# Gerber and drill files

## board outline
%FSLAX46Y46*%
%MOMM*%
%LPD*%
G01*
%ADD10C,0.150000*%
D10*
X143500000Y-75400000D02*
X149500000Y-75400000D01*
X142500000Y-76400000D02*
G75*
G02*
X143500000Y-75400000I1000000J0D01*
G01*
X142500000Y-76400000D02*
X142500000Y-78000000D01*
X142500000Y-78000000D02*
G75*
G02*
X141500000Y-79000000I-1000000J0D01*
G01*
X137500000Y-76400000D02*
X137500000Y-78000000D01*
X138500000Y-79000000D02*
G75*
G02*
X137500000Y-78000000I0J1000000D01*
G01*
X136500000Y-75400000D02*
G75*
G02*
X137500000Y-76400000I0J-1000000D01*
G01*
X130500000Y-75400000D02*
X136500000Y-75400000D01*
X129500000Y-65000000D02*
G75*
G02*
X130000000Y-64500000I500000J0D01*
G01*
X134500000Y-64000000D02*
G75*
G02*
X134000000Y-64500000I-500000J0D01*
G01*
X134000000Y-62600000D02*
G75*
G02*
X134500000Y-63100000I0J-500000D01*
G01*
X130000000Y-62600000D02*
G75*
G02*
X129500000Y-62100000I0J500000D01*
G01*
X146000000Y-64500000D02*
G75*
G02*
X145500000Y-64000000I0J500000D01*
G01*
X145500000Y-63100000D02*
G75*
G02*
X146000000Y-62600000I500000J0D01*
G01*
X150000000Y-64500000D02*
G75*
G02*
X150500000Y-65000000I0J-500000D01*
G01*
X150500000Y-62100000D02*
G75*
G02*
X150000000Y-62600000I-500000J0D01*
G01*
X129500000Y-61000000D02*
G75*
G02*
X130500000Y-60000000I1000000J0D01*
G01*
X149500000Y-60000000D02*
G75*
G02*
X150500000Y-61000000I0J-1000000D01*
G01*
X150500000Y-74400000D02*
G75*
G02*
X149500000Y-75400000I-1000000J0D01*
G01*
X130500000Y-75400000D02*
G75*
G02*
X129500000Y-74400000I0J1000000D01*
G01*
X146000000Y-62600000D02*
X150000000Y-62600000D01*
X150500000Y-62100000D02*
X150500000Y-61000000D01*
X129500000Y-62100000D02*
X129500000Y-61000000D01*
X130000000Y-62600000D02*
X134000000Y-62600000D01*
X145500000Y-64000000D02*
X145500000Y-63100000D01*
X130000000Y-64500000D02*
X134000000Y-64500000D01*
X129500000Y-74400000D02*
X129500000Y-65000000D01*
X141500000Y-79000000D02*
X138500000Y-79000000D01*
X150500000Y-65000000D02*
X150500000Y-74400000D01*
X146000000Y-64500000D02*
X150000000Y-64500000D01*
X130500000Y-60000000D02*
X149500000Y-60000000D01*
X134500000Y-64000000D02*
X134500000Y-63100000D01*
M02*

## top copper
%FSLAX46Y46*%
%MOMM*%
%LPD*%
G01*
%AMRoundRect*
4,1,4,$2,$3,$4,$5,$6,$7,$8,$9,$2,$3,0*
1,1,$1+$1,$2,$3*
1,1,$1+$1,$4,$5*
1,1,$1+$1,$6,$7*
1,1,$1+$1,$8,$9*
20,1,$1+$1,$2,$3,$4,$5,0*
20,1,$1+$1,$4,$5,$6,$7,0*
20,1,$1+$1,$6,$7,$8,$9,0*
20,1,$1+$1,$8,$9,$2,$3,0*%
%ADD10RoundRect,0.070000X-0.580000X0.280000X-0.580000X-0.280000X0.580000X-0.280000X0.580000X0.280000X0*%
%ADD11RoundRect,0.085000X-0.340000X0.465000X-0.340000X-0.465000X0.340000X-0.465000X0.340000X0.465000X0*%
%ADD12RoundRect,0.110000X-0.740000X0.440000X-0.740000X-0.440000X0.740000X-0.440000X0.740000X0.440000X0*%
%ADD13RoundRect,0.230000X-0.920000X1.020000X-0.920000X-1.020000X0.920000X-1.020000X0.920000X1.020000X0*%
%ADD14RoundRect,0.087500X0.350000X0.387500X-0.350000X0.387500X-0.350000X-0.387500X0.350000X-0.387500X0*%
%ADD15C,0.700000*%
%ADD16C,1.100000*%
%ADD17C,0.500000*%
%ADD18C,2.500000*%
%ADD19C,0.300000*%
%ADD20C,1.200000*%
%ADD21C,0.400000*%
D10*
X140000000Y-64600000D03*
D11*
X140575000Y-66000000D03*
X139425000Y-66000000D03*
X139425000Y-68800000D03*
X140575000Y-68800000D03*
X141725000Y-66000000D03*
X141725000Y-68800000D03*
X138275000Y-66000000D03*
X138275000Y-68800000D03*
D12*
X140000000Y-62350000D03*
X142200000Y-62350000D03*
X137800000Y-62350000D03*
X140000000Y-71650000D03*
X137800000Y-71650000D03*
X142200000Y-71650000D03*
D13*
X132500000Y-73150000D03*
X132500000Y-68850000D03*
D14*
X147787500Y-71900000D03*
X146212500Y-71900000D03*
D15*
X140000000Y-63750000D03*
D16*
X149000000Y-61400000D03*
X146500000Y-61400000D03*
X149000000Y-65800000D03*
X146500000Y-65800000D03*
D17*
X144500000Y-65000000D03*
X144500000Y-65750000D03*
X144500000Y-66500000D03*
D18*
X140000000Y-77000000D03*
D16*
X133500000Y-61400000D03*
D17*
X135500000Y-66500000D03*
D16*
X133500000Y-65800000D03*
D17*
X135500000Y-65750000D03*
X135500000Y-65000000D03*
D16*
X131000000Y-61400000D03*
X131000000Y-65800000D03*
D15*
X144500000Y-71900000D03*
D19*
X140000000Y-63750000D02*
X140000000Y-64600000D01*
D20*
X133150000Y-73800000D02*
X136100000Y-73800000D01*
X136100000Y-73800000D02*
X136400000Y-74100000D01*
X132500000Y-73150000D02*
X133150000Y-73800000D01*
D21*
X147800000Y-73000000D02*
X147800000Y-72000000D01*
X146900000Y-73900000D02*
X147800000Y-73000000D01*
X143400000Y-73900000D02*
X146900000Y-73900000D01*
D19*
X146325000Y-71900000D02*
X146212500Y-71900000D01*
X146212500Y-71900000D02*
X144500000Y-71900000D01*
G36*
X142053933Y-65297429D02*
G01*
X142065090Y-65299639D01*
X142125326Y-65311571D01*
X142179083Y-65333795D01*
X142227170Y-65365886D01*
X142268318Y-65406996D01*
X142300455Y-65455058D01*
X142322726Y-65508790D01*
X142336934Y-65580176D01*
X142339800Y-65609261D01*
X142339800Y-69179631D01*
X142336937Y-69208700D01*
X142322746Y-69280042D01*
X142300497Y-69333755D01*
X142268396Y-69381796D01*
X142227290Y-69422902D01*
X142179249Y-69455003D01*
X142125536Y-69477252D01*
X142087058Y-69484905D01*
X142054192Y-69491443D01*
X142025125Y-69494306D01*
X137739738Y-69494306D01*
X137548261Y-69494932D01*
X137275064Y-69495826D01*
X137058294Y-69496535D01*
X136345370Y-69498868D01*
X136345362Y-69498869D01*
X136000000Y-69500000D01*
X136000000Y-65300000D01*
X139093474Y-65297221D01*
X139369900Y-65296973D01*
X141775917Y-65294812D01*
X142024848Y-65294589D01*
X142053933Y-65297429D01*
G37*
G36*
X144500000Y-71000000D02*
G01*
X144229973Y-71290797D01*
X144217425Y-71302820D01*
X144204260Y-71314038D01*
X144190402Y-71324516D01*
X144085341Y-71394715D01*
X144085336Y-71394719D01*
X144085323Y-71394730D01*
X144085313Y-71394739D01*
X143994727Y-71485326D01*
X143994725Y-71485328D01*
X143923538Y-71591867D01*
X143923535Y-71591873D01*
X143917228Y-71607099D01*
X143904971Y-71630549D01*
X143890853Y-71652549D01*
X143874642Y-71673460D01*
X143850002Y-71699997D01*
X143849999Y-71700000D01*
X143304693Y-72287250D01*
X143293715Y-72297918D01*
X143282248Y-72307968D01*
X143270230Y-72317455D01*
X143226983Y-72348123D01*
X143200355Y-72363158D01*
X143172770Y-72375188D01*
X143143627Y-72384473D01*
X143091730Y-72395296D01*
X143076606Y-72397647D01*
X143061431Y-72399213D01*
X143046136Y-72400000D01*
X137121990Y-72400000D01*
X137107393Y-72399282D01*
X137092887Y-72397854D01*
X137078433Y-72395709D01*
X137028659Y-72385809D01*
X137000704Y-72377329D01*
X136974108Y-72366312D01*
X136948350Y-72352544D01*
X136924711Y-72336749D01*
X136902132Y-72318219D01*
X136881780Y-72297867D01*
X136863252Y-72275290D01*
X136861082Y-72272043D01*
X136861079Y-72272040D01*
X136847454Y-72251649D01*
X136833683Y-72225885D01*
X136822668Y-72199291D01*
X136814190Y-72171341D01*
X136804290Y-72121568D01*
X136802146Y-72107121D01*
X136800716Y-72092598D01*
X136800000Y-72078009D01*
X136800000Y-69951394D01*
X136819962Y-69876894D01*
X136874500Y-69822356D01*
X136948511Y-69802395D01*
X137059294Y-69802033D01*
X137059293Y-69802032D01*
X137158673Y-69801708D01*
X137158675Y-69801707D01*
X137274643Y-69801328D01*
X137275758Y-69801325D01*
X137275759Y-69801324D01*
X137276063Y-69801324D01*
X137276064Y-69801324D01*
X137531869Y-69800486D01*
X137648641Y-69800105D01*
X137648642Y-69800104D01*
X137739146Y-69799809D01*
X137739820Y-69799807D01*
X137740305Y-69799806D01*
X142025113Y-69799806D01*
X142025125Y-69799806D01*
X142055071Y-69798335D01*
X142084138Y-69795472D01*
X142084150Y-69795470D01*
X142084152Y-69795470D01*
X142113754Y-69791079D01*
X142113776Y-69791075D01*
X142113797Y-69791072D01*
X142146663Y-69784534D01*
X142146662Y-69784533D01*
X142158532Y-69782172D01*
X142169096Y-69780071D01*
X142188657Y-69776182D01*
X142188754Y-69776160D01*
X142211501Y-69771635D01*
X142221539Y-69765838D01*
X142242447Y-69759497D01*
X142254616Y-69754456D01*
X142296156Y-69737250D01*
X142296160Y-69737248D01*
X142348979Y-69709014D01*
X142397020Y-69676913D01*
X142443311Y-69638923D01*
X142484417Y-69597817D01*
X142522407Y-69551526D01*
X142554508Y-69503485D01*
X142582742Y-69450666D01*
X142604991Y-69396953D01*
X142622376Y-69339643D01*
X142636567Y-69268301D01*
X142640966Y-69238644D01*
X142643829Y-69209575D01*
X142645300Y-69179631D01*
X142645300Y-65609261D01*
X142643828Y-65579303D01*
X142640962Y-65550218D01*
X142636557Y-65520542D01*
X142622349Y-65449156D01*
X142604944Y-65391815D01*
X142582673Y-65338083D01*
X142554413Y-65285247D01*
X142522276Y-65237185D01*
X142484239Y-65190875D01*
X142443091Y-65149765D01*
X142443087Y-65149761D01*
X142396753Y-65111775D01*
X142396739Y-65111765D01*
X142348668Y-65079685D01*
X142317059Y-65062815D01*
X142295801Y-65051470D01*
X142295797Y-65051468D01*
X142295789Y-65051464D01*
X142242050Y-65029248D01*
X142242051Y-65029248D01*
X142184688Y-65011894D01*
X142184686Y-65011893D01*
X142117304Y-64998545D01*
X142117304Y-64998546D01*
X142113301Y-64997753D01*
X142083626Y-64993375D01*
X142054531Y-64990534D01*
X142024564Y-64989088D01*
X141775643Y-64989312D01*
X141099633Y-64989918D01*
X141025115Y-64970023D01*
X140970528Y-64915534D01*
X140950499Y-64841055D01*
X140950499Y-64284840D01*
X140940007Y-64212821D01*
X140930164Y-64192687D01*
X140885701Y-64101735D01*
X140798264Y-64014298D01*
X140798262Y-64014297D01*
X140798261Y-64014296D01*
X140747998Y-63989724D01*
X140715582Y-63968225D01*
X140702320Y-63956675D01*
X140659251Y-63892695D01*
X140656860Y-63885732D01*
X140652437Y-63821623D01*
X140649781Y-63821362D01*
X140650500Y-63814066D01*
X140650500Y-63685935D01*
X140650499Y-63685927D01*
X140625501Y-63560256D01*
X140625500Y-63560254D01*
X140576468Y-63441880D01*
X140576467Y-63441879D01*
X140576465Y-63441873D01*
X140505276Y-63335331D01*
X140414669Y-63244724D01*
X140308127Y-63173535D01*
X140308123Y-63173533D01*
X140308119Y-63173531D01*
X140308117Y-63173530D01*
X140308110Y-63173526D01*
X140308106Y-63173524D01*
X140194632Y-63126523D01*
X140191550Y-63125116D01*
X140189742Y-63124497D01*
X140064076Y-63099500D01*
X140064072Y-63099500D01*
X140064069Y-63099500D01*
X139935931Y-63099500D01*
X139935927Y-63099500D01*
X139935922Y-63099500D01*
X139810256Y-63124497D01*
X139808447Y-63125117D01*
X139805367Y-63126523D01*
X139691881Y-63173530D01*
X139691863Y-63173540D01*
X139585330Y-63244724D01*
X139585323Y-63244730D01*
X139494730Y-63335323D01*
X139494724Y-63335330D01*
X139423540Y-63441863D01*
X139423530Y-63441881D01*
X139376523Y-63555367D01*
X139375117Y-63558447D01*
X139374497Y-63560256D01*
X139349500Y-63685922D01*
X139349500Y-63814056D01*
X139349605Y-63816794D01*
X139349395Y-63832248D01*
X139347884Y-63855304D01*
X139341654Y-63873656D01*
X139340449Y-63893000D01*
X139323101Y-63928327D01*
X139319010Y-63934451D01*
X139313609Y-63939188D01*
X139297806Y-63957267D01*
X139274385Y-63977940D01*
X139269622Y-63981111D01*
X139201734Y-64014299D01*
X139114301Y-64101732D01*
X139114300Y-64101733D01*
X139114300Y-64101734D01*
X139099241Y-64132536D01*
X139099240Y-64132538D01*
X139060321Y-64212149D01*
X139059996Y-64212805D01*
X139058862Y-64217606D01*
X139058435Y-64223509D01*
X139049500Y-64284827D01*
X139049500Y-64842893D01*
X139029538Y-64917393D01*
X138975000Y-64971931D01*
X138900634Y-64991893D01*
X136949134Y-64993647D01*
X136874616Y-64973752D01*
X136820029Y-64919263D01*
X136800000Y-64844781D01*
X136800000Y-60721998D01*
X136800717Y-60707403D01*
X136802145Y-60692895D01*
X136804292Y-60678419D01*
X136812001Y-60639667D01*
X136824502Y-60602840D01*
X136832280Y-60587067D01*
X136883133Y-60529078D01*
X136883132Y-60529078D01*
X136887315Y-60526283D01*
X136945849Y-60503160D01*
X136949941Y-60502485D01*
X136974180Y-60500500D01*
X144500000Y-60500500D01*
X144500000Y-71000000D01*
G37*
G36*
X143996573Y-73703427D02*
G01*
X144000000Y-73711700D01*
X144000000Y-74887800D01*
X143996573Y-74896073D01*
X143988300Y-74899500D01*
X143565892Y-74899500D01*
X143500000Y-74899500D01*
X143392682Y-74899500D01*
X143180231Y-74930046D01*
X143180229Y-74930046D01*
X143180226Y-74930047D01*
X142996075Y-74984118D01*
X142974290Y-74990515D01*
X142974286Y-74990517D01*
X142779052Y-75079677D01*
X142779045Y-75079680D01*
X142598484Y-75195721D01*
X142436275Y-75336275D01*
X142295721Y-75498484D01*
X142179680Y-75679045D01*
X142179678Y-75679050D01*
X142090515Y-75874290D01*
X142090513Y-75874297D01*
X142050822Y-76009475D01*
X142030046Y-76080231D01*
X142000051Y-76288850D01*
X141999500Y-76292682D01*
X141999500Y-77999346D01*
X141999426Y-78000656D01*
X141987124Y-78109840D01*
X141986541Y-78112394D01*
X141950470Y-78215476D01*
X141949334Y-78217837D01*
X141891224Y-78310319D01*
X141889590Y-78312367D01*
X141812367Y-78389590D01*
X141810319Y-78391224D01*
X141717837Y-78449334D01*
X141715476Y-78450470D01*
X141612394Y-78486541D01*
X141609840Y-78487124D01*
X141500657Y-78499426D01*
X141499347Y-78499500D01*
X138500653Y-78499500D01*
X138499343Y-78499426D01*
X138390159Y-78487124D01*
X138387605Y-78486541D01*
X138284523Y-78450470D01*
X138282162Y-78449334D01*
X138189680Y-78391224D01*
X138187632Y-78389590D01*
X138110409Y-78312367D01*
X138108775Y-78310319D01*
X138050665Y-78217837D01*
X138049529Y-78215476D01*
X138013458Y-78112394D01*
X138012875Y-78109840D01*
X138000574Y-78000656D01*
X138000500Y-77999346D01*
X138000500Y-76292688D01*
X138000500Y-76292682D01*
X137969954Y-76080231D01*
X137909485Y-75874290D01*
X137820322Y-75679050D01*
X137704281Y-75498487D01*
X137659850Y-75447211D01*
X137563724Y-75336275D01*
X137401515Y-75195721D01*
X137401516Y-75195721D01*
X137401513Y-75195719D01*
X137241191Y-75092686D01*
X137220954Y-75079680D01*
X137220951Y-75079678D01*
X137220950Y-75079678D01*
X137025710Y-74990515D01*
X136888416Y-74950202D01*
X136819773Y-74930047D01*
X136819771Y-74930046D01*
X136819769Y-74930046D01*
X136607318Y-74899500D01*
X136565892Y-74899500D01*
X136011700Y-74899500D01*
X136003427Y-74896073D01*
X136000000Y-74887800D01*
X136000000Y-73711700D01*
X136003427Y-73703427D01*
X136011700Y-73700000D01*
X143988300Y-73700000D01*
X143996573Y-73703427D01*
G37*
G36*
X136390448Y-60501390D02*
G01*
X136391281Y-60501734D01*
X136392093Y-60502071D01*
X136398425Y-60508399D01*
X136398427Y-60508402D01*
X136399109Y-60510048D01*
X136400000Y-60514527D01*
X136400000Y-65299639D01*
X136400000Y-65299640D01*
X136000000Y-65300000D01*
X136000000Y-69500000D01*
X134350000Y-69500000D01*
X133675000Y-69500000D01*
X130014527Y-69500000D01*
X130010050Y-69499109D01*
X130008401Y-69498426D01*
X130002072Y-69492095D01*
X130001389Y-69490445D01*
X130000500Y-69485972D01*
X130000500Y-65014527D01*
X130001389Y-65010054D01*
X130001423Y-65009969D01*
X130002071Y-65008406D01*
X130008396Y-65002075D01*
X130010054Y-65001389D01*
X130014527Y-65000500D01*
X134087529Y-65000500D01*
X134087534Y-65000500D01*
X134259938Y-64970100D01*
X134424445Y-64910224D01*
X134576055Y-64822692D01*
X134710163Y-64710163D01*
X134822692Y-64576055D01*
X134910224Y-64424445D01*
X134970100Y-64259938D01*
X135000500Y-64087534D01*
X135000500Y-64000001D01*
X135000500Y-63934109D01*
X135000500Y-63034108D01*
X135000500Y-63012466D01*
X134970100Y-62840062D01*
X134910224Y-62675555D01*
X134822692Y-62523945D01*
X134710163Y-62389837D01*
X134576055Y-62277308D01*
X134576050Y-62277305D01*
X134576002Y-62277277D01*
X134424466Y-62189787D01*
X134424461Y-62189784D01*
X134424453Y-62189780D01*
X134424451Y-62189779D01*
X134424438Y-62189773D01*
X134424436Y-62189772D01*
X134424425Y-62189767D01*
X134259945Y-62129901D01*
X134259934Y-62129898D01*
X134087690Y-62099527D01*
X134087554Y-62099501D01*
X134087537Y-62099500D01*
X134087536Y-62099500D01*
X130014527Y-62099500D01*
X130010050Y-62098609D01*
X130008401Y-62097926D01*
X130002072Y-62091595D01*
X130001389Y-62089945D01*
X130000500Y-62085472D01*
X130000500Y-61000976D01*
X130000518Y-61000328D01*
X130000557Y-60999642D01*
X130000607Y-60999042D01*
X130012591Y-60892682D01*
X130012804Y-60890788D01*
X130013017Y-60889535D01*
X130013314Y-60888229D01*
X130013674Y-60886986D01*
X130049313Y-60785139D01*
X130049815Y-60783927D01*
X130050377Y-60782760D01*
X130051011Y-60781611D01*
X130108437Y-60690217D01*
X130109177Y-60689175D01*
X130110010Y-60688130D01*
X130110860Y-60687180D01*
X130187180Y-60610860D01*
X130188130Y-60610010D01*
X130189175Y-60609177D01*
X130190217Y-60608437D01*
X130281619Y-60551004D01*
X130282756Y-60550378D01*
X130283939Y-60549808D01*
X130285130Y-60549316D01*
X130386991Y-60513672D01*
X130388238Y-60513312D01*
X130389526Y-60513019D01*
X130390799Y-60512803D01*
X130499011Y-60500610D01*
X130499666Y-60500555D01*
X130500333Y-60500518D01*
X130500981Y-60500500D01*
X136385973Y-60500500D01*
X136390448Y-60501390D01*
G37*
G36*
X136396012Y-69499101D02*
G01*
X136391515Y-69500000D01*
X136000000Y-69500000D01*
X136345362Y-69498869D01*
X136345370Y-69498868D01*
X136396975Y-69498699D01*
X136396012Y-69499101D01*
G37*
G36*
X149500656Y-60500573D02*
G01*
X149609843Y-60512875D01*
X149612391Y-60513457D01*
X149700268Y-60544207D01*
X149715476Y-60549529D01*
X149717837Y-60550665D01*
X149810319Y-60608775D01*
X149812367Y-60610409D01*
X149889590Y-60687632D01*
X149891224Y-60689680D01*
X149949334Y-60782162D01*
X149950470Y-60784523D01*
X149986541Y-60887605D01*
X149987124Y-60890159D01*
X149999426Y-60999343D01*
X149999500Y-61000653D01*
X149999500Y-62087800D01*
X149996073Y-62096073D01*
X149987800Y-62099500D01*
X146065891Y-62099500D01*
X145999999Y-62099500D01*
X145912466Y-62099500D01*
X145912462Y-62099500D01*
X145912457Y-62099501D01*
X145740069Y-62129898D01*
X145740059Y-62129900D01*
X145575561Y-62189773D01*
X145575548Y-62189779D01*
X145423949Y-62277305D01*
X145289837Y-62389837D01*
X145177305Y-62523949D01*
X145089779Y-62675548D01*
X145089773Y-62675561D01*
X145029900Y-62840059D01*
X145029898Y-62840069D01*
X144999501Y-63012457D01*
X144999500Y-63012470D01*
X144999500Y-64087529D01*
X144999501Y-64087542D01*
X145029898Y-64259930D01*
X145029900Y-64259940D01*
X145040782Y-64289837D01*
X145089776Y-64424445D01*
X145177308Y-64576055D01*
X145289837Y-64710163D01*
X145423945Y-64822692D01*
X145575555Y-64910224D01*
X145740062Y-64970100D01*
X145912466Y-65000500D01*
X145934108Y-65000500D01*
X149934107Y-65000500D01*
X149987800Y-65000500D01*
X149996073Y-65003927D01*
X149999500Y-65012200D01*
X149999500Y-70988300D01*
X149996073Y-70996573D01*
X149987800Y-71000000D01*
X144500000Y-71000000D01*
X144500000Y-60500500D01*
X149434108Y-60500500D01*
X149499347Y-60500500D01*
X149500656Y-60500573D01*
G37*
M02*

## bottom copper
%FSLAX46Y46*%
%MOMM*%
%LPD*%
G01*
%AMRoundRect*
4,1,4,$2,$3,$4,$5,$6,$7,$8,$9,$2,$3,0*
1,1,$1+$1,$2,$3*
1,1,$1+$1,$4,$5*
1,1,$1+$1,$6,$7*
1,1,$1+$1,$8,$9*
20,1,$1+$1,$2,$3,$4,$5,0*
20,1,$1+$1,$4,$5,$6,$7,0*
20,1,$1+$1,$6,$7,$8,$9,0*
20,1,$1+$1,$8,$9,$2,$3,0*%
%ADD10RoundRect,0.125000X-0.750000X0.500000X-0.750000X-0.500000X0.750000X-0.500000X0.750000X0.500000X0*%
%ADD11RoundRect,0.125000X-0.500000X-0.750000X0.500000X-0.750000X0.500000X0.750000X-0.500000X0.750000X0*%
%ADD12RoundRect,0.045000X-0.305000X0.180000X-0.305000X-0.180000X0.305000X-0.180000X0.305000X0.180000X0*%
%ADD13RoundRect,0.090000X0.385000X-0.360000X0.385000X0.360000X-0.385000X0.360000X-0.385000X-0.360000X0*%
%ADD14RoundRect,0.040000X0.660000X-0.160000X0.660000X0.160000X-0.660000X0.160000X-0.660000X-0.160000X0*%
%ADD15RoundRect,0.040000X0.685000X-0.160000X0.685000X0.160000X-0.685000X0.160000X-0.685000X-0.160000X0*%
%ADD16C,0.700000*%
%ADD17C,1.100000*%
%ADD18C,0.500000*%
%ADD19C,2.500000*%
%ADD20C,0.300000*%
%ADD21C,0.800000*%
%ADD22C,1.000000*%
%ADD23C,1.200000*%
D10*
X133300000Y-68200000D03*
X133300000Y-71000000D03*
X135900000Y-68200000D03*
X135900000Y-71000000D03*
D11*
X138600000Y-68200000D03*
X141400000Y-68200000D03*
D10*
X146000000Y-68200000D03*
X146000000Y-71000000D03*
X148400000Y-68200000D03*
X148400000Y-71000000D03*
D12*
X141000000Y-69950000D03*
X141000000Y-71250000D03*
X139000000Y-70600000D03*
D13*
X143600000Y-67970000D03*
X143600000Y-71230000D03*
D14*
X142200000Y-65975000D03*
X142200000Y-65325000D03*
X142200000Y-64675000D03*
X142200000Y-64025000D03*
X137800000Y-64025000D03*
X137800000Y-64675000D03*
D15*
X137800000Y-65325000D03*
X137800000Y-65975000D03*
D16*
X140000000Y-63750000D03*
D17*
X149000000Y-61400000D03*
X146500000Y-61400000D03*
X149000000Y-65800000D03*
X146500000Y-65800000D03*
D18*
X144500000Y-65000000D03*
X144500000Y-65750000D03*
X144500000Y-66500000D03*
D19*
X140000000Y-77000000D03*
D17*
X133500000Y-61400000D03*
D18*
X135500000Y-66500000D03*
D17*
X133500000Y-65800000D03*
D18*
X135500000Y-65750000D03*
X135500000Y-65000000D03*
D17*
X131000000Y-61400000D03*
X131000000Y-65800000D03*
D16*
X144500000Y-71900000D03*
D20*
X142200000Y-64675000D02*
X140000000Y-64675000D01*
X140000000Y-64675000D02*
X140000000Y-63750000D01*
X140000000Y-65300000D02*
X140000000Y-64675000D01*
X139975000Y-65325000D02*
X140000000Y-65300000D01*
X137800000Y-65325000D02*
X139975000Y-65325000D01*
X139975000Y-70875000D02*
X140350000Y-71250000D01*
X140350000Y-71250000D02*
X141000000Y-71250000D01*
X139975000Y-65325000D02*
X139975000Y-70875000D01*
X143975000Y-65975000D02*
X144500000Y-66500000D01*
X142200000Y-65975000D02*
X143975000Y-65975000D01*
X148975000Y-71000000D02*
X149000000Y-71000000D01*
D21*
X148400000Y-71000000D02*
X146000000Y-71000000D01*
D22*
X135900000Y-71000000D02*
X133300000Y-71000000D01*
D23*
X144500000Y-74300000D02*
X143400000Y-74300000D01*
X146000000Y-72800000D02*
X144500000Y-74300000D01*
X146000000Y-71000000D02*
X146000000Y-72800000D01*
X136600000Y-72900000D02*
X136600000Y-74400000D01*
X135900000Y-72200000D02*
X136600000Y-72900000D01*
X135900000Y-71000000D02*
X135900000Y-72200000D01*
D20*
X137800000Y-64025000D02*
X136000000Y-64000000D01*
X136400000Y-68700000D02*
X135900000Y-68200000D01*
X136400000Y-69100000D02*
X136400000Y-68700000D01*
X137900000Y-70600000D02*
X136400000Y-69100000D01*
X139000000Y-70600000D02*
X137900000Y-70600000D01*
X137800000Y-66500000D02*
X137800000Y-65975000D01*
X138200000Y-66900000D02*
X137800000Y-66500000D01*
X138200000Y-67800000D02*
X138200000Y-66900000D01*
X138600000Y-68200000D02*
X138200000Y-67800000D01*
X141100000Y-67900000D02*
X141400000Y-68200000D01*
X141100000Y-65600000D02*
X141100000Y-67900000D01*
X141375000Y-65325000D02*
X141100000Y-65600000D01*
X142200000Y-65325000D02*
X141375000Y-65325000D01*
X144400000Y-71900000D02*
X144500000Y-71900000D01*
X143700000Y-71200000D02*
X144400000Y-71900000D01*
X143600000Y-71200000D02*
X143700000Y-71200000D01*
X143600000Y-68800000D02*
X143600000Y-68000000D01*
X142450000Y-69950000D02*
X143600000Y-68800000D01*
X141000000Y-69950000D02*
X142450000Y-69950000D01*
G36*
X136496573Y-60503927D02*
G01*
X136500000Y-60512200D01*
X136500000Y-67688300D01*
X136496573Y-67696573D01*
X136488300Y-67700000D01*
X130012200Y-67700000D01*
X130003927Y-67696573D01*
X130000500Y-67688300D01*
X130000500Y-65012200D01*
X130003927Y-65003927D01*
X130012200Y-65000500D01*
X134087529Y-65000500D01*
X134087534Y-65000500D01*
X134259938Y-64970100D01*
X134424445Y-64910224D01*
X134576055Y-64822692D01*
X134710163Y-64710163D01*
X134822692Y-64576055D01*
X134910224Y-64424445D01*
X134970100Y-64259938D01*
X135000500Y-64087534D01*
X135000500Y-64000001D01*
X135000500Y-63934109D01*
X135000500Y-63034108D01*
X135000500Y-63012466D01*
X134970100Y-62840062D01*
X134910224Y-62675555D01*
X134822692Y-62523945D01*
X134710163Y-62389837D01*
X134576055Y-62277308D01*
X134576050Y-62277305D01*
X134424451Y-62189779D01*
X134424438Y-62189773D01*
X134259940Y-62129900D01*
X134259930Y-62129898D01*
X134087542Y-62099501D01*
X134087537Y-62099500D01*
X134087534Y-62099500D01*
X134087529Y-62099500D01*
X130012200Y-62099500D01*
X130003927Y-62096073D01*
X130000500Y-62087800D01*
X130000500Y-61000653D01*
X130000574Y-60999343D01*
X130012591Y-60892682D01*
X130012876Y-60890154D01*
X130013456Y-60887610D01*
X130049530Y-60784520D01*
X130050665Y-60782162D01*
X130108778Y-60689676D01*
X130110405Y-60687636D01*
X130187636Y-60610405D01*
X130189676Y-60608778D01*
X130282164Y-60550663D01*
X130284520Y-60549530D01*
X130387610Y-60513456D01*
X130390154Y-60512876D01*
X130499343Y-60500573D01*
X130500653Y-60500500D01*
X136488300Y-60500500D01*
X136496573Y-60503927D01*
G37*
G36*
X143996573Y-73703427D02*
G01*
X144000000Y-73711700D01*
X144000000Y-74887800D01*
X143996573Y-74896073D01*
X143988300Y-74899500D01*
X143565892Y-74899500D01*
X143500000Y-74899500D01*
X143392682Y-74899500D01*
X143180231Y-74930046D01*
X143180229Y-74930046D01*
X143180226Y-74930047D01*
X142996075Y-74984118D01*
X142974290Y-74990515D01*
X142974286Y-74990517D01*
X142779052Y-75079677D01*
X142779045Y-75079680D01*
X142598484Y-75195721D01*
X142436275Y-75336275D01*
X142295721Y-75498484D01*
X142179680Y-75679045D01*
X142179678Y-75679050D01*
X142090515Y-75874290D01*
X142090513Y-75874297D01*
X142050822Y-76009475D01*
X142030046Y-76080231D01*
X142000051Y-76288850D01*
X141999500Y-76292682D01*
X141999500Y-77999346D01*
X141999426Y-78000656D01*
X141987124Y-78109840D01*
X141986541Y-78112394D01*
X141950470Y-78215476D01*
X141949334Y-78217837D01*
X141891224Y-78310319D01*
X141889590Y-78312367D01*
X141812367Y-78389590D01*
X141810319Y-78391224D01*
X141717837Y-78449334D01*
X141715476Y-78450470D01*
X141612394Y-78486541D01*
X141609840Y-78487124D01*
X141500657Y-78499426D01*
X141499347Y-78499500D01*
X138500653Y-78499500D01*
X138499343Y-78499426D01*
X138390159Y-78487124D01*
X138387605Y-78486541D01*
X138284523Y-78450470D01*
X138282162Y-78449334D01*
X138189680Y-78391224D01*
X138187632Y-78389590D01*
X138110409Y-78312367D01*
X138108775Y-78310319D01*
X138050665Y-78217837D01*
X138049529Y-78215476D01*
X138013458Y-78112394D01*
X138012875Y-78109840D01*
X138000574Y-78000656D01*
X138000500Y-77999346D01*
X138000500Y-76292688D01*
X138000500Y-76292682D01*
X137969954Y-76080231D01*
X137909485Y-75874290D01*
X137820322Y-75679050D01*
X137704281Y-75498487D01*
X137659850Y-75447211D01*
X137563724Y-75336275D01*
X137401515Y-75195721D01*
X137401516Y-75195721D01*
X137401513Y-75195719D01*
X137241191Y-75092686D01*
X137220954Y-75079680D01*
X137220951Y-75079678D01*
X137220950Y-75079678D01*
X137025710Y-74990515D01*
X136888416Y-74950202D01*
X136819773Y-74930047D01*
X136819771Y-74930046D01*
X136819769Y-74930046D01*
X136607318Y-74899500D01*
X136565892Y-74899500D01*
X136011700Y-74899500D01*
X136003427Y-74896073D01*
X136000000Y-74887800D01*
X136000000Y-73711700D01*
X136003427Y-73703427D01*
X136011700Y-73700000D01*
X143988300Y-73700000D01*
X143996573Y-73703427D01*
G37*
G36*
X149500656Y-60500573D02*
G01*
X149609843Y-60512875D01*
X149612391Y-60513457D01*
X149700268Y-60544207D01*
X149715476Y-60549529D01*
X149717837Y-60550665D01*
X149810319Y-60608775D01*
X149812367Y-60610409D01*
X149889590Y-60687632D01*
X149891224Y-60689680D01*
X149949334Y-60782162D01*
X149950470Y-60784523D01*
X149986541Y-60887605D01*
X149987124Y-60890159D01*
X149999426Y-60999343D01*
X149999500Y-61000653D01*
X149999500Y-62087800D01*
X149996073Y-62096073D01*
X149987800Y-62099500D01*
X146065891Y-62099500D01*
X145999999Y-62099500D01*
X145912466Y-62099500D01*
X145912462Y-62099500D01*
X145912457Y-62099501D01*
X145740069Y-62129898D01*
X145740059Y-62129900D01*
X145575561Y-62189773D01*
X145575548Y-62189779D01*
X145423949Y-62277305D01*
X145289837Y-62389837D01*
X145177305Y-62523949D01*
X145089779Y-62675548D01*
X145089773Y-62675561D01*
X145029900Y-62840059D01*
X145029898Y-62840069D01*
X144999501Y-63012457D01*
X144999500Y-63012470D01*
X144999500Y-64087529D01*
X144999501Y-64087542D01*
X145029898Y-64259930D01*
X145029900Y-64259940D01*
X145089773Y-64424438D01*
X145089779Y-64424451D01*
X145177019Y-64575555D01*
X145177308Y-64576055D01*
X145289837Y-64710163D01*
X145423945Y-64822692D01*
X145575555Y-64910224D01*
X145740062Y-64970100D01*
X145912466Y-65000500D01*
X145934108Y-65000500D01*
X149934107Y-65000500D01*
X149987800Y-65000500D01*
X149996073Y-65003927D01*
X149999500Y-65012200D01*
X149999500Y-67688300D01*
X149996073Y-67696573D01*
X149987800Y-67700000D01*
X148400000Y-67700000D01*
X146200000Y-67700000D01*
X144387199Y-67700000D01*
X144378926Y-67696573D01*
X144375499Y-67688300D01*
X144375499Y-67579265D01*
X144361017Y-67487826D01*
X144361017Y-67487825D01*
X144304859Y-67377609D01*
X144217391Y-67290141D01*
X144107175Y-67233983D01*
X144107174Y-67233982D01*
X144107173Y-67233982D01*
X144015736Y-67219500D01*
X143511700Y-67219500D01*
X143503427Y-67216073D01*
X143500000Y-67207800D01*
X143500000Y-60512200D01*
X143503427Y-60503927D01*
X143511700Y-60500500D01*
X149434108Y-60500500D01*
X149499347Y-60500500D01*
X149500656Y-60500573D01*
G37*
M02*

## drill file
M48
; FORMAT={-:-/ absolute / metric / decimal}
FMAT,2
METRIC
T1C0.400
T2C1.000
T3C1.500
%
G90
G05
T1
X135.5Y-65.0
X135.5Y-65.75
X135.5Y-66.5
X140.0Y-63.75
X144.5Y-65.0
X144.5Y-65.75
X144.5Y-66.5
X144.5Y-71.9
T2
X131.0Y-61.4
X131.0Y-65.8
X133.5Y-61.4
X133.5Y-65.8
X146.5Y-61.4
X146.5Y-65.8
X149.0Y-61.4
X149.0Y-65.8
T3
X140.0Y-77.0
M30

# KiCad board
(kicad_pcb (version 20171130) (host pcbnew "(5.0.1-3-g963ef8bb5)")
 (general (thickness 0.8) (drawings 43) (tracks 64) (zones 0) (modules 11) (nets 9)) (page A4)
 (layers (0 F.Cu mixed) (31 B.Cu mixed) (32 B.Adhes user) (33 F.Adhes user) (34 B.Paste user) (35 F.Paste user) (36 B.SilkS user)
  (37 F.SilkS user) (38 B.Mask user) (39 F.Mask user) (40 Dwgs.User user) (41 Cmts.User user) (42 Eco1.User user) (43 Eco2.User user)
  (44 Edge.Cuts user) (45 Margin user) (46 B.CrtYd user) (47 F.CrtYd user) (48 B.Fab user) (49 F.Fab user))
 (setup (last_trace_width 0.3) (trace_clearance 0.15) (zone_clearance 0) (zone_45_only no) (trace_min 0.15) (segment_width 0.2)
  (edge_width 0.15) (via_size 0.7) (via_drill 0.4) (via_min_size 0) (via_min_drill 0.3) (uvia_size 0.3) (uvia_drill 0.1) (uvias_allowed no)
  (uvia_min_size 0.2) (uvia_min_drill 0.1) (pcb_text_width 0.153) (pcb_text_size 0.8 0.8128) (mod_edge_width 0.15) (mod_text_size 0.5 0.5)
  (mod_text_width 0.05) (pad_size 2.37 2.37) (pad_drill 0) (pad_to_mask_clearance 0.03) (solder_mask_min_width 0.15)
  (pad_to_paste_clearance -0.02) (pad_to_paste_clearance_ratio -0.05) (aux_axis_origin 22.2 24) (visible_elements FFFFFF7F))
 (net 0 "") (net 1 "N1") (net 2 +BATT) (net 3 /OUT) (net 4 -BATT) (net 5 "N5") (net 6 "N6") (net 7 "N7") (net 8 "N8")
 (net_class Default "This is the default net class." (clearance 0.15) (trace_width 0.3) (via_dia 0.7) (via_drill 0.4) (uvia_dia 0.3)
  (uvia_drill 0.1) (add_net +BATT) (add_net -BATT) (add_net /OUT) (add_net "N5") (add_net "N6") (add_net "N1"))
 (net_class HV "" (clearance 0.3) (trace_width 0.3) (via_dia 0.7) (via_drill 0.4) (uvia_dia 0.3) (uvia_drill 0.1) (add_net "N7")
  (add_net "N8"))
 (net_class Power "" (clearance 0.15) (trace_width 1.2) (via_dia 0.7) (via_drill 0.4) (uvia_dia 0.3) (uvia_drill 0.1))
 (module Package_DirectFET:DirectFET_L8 (layer F.Cu) (at 140 67 270)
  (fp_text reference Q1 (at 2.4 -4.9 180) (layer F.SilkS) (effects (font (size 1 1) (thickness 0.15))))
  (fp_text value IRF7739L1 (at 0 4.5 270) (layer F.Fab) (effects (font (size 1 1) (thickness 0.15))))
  (pad 2 smd roundrect (at -2.4 0 270) (size 0.7 1.3) (layers F.Cu F.Paste F.Mask) (roundrect_rratio 0.1) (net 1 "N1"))
  (pad 3 smd roundrect (at -1 -0.575 270) (size 1.1 0.85) (layers F.Cu F.Paste F.Mask) (roundrect_rratio 0.1) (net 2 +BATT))
  (pad 3 smd roundrect (at -1 0.575 270) (size 1.1 0.85) (layers F.Cu F.Paste F.Mask) (roundrect_rratio 0.1) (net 2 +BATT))
  (pad 3 smd roundrect (at 1.8 0.575 270) (size 1.1 0.85) (layers F.Cu F.Paste F.Mask) (roundrect_rratio 0.1) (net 2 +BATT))
  (pad 3 smd roundrect (at 1.8 -0.575 270) (size 1.1 0.85) (layers F.Cu F.Paste F.Mask) (roundrect_rratio 0.1) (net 2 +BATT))
  (pad 3 smd roundrect (at -1 -1.725 270) (size 1.1 0.85) (layers F.Cu F.Paste F.Mask) (roundrect_rratio 0.1) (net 2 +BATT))
  (pad 3 smd roundrect (at 1.8 -1.725 270) (size 1.1 0.85) (layers F.Cu F.Paste F.Mask) (roundrect_rratio 0.1) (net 2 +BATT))
  (pad 3 smd roundrect (at -1 1.725 270) (size 1.1 0.85) (layers F.Cu F.Paste F.Mask) (roundrect_rratio 0.1) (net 2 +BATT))
  (pad 3 smd roundrect (at 1.8 1.725 270) (size 1.1 0.85) (layers F.Cu F.Paste F.Mask) (roundrect_rratio 0.1) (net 2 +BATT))
  (pad 1 smd roundrect (at -4.65 0 270) (size 1.1 1.7) (layers F.Cu F.Paste F.Mask) (roundrect_rratio 0.1) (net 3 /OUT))
  (pad 1 smd roundrect (at -4.65 -2.2 270) (size 1.1 1.7) (layers F.Cu F.Paste F.Mask) (roundrect_rratio 0.1) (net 3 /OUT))
  (pad 1 smd roundrect (at -4.65 2.2 270) (size 1.1 1.7) (layers F.Cu F.Paste F.Mask) (roundrect_rratio 0.1) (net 3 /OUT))
  (pad 1 smd roundrect (at 4.65 0 270) (size 1.1 1.7) (layers F.Cu F.Paste F.Mask) (roundrect_rratio 0.1) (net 3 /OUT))
  (pad 1 smd roundrect (at 4.65 2.2 270) (size 1.1 1.7) (layers F.Cu F.Paste F.Mask) (roundrect_rratio 0.1) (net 3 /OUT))
  (pad 1 smd roundrect (at 4.65 -2.2 270) (size 1.1 1.7) (layers F.Cu F.Paste F.Mask) (roundrect_rratio 0.1) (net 3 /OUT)))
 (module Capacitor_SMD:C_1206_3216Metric (layer B.Cu) (at 133.3 69.6 270)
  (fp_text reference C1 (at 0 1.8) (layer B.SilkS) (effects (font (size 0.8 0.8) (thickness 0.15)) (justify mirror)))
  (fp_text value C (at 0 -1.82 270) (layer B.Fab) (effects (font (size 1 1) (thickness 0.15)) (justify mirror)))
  (pad 1 smd roundrect (at -1.4 0 270) (size 1.25 1.75) (layers B.Cu B.Paste B.Mask) (roundrect_rratio 0.1) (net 2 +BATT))
  (pad 2 smd roundrect (at 1.4 0 270) (size 1.25 1.75) (layers B.Cu B.Paste B.Mask) (roundrect_rratio 0.1) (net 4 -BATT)))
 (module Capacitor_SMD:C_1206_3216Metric (layer B.Cu) (at 135.9 69.6 270)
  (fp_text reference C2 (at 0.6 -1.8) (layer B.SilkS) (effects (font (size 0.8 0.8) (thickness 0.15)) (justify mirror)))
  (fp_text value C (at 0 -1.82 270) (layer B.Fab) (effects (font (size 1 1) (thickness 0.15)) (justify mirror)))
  (pad 1 smd roundrect (at -1.4 0 270) (size 1.25 1.75) (layers B.Cu B.Paste B.Mask) (roundrect_rratio 0.1) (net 2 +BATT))
  (pad 2 smd roundrect (at 1.4 0 270) (size 1.25 1.75) (layers B.Cu B.Paste B.Mask) (roundrect_rratio 0.1) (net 4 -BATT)))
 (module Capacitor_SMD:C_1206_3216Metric (layer B.Cu) (at 140 68.2)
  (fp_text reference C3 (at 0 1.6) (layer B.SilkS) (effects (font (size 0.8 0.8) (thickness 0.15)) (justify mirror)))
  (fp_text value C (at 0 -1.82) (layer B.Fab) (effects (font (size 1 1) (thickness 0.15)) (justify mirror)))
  (pad 1 smd roundrect (at -1.4 0) (size 1.25 1.75) (layers B.Cu B.Paste B.Mask) (roundrect_rratio 0.1) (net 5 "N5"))
  (pad 2 smd roundrect (at 1.4 0) (size 1.25 1.75) (layers B.Cu B.Paste B.Mask) (roundrect_rratio 0.1) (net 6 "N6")))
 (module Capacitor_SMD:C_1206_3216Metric (layer B.Cu) (at 146 69.6 270)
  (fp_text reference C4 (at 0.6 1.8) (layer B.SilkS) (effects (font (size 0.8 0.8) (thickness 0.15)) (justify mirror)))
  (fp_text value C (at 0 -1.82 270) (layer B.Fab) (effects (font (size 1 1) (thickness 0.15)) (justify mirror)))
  (pad 1 smd roundrect (at -1.4 0 270) (size 1.25 1.75) (layers B.Cu B.Paste B.Mask) (roundrect_rratio 0.1) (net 3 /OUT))
  (pad 2 smd roundrect (at 1.4 0 270) (size 1.25 1.75) (layers B.Cu B.Paste B.Mask) (roundrect_rratio 0.1) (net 4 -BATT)))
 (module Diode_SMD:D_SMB (layer F.Cu) (at 132.5 71 270)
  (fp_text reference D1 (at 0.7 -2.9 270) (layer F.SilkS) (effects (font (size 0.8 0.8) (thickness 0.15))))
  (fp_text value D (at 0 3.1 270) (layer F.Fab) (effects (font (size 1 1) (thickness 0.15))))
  (pad 2 smd roundrect (at 2.15 0 270) (size 2.5 2.3) (layers F.Cu F.Paste F.Mask) (roundrect_rratio 0.1) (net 4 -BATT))
  (pad 1 smd roundrect (at -2.15 0 270) (size 2.5 2.3) (layers F.Cu F.Paste F.Mask) (roundrect_rratio 0.1) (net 2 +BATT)))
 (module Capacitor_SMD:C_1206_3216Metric (layer B.Cu) (at 148.4 69.6 270)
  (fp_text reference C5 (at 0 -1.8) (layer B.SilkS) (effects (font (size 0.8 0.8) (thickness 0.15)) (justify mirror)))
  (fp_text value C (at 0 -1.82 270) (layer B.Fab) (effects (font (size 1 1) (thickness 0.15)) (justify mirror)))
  (pad 1 smd roundrect (at -1.4 0 270) (size 1.25 1.75) (layers B.Cu B.Paste B.Mask) (roundrect_rratio 0.1) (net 3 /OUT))
  (pad 2 smd roundrect (at 1.4 0 270) (size 1.25 1.75) (layers B.Cu B.Paste B.Mask) (roundrect_rratio 0.1) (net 4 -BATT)))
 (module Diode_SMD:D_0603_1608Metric (layer F.Cu) (at 147 71.9 180)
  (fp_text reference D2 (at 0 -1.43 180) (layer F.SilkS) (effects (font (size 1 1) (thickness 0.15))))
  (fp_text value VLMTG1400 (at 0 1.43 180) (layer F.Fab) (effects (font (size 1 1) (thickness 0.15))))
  (pad 1 smd roundrect (at -0.7875 0 180) (size 0.875 0.95) (layers F.Cu F.Paste F.Mask) (roundrect_rratio 0.1) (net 4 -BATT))
  (pad 2 smd roundrect (at 0.7875 0 180) (size 0.875 0.95) (layers F.Cu F.Paste F.Mask) (roundrect_rratio 0.1) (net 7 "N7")))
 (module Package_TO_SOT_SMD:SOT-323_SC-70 (layer B.Cu) (at 140 70.6 180)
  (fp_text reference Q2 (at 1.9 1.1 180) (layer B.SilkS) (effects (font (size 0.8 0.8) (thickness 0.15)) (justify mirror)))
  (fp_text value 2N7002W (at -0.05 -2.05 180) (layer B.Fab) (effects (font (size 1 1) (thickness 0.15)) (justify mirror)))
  (pad 1 smd roundrect (at -1 0.65 270) (size 0.45 0.7) (layers B.Cu B.Paste B.Mask) (roundrect_rratio 0.1) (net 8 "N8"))
  (pad 2 smd roundrect (at -1 -0.65 270) (size 0.45 0.7) (layers B.Cu B.Paste B.Mask) (roundrect_rratio 0.1) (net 1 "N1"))
  (pad 3 smd roundrect (at 1 0 270) (size 0.45 0.7) (layers B.Cu B.Paste B.Mask) (roundrect_rratio 0.1) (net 2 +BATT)))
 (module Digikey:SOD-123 (layer B.Cu) (at 143.6 69.6 90)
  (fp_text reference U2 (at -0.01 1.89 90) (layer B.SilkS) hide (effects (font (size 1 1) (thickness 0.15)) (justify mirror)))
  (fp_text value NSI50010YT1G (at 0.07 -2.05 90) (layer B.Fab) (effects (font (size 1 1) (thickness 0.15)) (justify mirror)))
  (pad A smd roundrect (at 1.63 0 90) (size 0.9 0.95) (layers B.Cu B.Paste B.Mask) (roundrect_rratio 0.1) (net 8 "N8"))
  (pad K smd roundrect (at -1.63 0 90) (size 0.9 0.95) (layers B.Cu B.Paste B.Mask) (roundrect_rratio 0.1) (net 7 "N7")))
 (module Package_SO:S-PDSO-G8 (layer B.Cu) (at 140 65)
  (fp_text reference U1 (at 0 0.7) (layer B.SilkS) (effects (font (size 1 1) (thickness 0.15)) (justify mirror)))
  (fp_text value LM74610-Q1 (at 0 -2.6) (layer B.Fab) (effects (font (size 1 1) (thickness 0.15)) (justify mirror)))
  (pad 8 smd roundrect (at 2.2 0.975 90) (size 0.4 1.4) (layers B.Cu B.Paste B.Mask) (roundrect_rratio 0.1) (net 3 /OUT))
  (pad 7 smd roundrect (at 2.2 0.325 90) (size 0.4 1.4) (layers B.Cu B.Paste B.Mask) (roundrect_rratio 0.1) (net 6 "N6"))
  (pad 6 smd roundrect (at 2.2 -0.325 90) (size 0.4 1.4) (layers B.Cu B.Paste B.Mask) (roundrect_rratio 0.1) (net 1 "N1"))
  (pad 5 smd roundrect (at 2.2 -0.975 90) (size 0.4 1.4) (layers B.Cu B.Paste B.Mask) (roundrect_rratio 0.1))
  (pad 4 smd roundrect (at -2.2 -0.975 90) (size 0.4 1.4) (layers B.Cu B.Paste B.Mask) (roundrect_rratio 0.1) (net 2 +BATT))
  (pad 3 smd roundrect (at -2.2 -0.325 90) (size 0.4 1.4) (layers B.Cu B.Paste B.Mask) (roundrect_rratio 0.1))
  (pad 2 smd roundrect (at -2.2 0.325 90) (size 0.4 1.45) (layers B.Cu B.Paste B.Mask) (roundrect_rratio 0.1) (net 1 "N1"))
  (pad 1 smd roundrect (at -2.2 0.975 90) (size 0.4 1.45) (layers B.Cu B.Paste B.Mask) (roundrect_rratio 0.1) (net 5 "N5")))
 (gr_line (start 143.5 75.4) (end 149.5 75.4) (layer Edge.Cuts) (width 0.15))
 (gr_arc (start 143.5 76.4) (end 143.5 75.4) (angle -90) (layer Edge.Cuts) (width 0.15))
 (gr_line (start 142.5 76.4) (end 142.5 78) (layer Edge.Cuts) (width 0.15))
 (gr_arc (start 141.5 78) (end 141.5 79) (angle -90) (layer Edge.Cuts) (width 0.15))
 (gr_line (start 137.5 76.4) (end 137.5 78) (layer Edge.Cuts) (width 0.15))
 (gr_arc (start 138.5 78) (end 137.5 78) (angle -90) (layer Edge.Cuts) (width 0.15))
 (gr_arc (start 136.5 76.4) (end 137.5 76.4) (angle -90) (layer Edge.Cuts) (width 0.15))
 (gr_line (start 130.5 75.4) (end 136.5 75.4) (layer Edge.Cuts) (width 0.15))
 (gr_arc (start 130 65) (end 130 64.5) (angle -90) (layer Edge.Cuts) (width 0.15))
 (gr_arc (start 134 64) (end 134 64.5) (angle -90) (layer Edge.Cuts) (width 0.15))
 (gr_arc (start 134 63.1) (end 134.5 63.1) (angle -90) (layer Edge.Cuts) (width 0.15))
 (gr_arc (start 130 62.1) (end 129.5 62.1) (angle -90) (layer Edge.Cuts) (width 0.15))
 (gr_arc (start 146 64) (end 145.5 64) (angle -90) (layer Edge.Cuts) (width 0.15))
 (gr_arc (start 146 63.1) (end 146 62.6) (angle -90) (layer Edge.Cuts) (width 0.15))
 (gr_arc (start 150 65) (end 150.5 65) (angle -90) (layer Edge.Cuts) (width 0.15))
 (gr_arc (start 150 62.1) (end 150 62.6) (angle -90) (layer Edge.Cuts) (width 0.15))
 (gr_arc (start 130.5 61) (end 130.5 60) (angle -90) (layer Edge.Cuts) (width 0.15))
 (gr_arc (start 149.5 61) (end 150.5 61) (angle -90) (layer Edge.Cuts) (width 0.15))
 (gr_arc (start 149.5 74.4) (end 149.5 75.4) (angle -90) (layer Edge.Cuts) (width 0.15))
 (gr_arc (start 130.5 74.4) (end 129.5 74.4) (angle -90) (layer Edge.Cuts) (width 0.15))
 (gr_line (start 146 62.6) (end 150 62.6) (layer Edge.Cuts) (width 0.15))
 (gr_line (start 150.5 62.1) (end 150.5 61) (layer Edge.Cuts) (width 0.15))
 (gr_line (start 129.5 62.1) (end 129.5 61) (layer Edge.Cuts) (width 0.15))
 (gr_line (start 130 62.6) (end 134 62.6) (layer Edge.Cuts) (width 0.15))
 (gr_line (start 145.5 64) (end 145.5 63.1) (layer Edge.Cuts) (width 0.15))
 (gr_line (start 130 64.5) (end 134 64.5) (layer Edge.Cuts) (width 0.15))
 (gr_line (start 129.5 74.4) (end 129.5 65) (layer Edge.Cuts) (width 0.15))
 (gr_line (start 141.5 79) (end 138.5 79) (layer Edge.Cuts) (width 0.15))
 (gr_line (start 150.5 65) (end 150.5 74.4) (layer Edge.Cuts) (width 0.15))
 (gr_line (start 146 64.5) (end 150 64.5) (layer Edge.Cuts) (width 0.15))
 (gr_line (start 130.5 60) (end 149.5 60) (layer Edge.Cuts) (width 0.15))
 (gr_line (start 134.5 64) (end 134.5 63.1) (layer Edge.Cuts) (width 0.15))
 (via (at 140 63.75) (size 0.7) (drill 0.4) (layers F.Cu B.Cu) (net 1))
 (segment (start 142.2 64.675) (end 140 64.675) (width 0.3) (layer B.Cu) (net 1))
 (segment (start 140 64.675) (end 140 63.75) (width 0.3) (layer B.Cu) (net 1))
 (segment (start 140 63.75) (end 140 64.6) (width 0.3) (layer F.Cu) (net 1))
 (segment (start 140 65.3) (end 140 64.675) (width 0.3) (layer B.Cu) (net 1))
 (segment (start 139.975 65.325) (end 140 65.3) (width 0.3) (layer B.Cu) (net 1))
 (segment (start 137.8 65.325) (end 139.975 65.325) (width 0.3) (layer B.Cu) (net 1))
 (segment (start 139.975 70.875) (end 140.35 71.25) (width 0.3) (layer B.Cu) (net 1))
 (segment (start 140.35 71.25) (end 141 71.25) (width 0.3) (layer B.Cu) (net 1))
 (segment (start 139.975 65.325) (end 139.975 70.875) (width 0.3) (layer B.Cu) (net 1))
 (via (at 149 61.4) (size 1.1) (drill 1) (layers F.Cu B.Cu) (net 3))
 (via (at 146.5 61.4) (size 1.1) (drill 1) (layers F.Cu B.Cu) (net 3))
 (via (at 149 65.8) (size 1.1) (drill 1) (layers F.Cu B.Cu) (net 3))
 (via (at 146.5 65.8) (size 1.1) (drill 1) (layers F.Cu B.Cu) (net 3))
 (segment (start 143.975 65.975) (end 144.5 66.5) (width 0.3) (layer B.Cu) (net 3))
 (segment (start 142.2 65.975) (end 143.975 65.975) (width 0.3) (layer B.Cu) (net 3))
 (via (at 144.5 65) (size 0.5) (drill 0.4) (layers F.Cu B.Cu) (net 3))
 (via (at 144.5 65.75) (size 0.5) (drill 0.4) (layers F.Cu B.Cu) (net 3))
 (via (at 144.5 66.5) (size 0.5) (drill 0.4) (layers F.Cu B.Cu) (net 3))
 (via (at 140 77) (size 2.5) (drill 1.5) (layers F.Cu B.Cu) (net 4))
 (segment (start 148.975 71) (end 149 71) (width 0.3) (layer B.Cu) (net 4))
 (segment (start 148.4 71) (end 146 71) (width 0.8) (layer B.Cu) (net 4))
 (segment (start 135.9 71) (end 133.3 71) (width 1) (layer B.Cu) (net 4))
 (segment (start 133.15 73.8) (end 136.1 73.8) (width 1.2) (layer F.Cu) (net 4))
 (segment (start 136.1 73.8) (end 136.4 74.1) (width 1.2) (layer F.Cu) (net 4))
 (segment (start 132.5 73.15) (end 133.15 73.8) (width 1.2) (layer F.Cu) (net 4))
 (segment (start 147.8 73) (end 147.8 72) (width 0.4) (layer F.Cu) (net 4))
 (segment (start 146.9 73.9) (end 147.8 73) (width 0.4) (layer F.Cu) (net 4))
 (segment (start 143.4 73.9) (end 146.9 73.9) (width 0.4) (layer F.Cu) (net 4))
 (segment (start 144.5 74.3) (end 143.4 74.3) (width 1.2) (layer B.Cu) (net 4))
 (segment (start 146 72.8) (end 144.5 74.3) (width 1.2) (layer B.Cu) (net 4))
 (segment (start 146 71) (end 146 72.8) (width 1.2) (layer B.Cu) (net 4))
 (segment (start 136.6 72.9) (end 136.6 74.4) (width 1.2) (layer B.Cu) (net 4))
 (segment (start 135.9 72.2) (end 136.6 72.9) (width 1.2) (layer B.Cu) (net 4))
 (segment (start 135.9 71) (end 135.9 72.2) (width 1.2) (layer B.Cu) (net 4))
 (via (at 133.5 61.4) (size 1.1) (drill 1) (layers F.Cu B.Cu) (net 2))
 (via (at 135.5 66.5) (size 0.5) (drill 0.4) (layers F.Cu B.Cu) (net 2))
 (via (at 133.5 65.8) (size 1.1) (drill 1) (layers F.Cu B.Cu) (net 2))
 (via (at 135.5 65.75) (size 0.5) (drill 0.4) (layers F.Cu B.Cu) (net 2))
 (via (at 135.5 65) (size 0.5) (drill 0.4) (layers F.Cu B.Cu) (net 2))
 (segment (start 137.8 64.025) (end 136 64) (width 0.3) (layer B.Cu) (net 2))
 (via (at 131 61.4) (size 1.1) (drill 1) (layers F.Cu B.Cu) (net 2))
 (via (at 131 65.8) (size 1.1) (drill 1) (layers F.Cu B.Cu) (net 2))
 (segment (start 136.4 68.7) (end 135.9 68.2) (width 0.3) (layer B.Cu) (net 2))
 (segment (start 136.4 69.1) (end 136.4 68.7) (width 0.3) (layer B.Cu) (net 2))
 (segment (start 137.9 70.6) (end 136.4 69.1) (width 0.3) (layer B.Cu) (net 2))
 (segment (start 139 70.6) (end 137.9 70.6) (width 0.3) (layer B.Cu) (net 2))
 (segment (start 137.8 66.5) (end 137.8 65.975) (width 0.3) (layer B.Cu) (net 5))
 (segment (start 138.2 66.9) (end 137.8 66.5) (width 0.3) (layer B.Cu) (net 5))
 (segment (start 138.2 67.8) (end 138.2 66.9) (width 0.3) (layer B.Cu) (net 5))
 (segment (start 138.6 68.2) (end 138.2 67.8) (width 0.3) (layer B.Cu) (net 5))
 (segment (start 141.1 67.9) (end 141.4 68.2) (width 0.3) (layer B.Cu) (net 6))
 (segment (start 141.1 65.6) (end 141.1 67.9) (width 0.3) (layer B.Cu) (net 6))
 (segment (start 141.375 65.325) (end 141.1 65.6) (width 0.3) (layer B.Cu) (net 6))
 (segment (start 142.2 65.325) (end 141.375 65.325) (width 0.3) (layer B.Cu) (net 6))
 (via (at 144.5 71.9) (size 0.7) (drill 0.4) (layers F.Cu B.Cu) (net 7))
 (segment (start 146.325 71.9) (end 146.2125 71.9) (width 0.3) (layer F.Cu) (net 7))
 (segment (start 146.2125 71.9) (end 144.5 71.9) (width 0.3) (layer F.Cu) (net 7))
 (segment (start 144.4 71.9) (end 144.5 71.9) (width 0.3) (layer B.Cu) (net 7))
 (segment (start 143.7 71.2) (end 144.4 71.9) (width 0.3) (layer B.Cu) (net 7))
 (segment (start 143.6 71.2) (end 143.7 71.2) (width 0.3) (layer B.Cu) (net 7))
 (segment (start 143.6 68.8) (end 143.6 68) (width 0.3) (layer B.Cu) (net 8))
 (segment (start 142.45 69.95) (end 143.6 68.8) (width 0.3) (layer B.Cu) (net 8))
 (segment (start 141 69.95) (end 142.45 69.95) (width 0.3) (layer B.Cu) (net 8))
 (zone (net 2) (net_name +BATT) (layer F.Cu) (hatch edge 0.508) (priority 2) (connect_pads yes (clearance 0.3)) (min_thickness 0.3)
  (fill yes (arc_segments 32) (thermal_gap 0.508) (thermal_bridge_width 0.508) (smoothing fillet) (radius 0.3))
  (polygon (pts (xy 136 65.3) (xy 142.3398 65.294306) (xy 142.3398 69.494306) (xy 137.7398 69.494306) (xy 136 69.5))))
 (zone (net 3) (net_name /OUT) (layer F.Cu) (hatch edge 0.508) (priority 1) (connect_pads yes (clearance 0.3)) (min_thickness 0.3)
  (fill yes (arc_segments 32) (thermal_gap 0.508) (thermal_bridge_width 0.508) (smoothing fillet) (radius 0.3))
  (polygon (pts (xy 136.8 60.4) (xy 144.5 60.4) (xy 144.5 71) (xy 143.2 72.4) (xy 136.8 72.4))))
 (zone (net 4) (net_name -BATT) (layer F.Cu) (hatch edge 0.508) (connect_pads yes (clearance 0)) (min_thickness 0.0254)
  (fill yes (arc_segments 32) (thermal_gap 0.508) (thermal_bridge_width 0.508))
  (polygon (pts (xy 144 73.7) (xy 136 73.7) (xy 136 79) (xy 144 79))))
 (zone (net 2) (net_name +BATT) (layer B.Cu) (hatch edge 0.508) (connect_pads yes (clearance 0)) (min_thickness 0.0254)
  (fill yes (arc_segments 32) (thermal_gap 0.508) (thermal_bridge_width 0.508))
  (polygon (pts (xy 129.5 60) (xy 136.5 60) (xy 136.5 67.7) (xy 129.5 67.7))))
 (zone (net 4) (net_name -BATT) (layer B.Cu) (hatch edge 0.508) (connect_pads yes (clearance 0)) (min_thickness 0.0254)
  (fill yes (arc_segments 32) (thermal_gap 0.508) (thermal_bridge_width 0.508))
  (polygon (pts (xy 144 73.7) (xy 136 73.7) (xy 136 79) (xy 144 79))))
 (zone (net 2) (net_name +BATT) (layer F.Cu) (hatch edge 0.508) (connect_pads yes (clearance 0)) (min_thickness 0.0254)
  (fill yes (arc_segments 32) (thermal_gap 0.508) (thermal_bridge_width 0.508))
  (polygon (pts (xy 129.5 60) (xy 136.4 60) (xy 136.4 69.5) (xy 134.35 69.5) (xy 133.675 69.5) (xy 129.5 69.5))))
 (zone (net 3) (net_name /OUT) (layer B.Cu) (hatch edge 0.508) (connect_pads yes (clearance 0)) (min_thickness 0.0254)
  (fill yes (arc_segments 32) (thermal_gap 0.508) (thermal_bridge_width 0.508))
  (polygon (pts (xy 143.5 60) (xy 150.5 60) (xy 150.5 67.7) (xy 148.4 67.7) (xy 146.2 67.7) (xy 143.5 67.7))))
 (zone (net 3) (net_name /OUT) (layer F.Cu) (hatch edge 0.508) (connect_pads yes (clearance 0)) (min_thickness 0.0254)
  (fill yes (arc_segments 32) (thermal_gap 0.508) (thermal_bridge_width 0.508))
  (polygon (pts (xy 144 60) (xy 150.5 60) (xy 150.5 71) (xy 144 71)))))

